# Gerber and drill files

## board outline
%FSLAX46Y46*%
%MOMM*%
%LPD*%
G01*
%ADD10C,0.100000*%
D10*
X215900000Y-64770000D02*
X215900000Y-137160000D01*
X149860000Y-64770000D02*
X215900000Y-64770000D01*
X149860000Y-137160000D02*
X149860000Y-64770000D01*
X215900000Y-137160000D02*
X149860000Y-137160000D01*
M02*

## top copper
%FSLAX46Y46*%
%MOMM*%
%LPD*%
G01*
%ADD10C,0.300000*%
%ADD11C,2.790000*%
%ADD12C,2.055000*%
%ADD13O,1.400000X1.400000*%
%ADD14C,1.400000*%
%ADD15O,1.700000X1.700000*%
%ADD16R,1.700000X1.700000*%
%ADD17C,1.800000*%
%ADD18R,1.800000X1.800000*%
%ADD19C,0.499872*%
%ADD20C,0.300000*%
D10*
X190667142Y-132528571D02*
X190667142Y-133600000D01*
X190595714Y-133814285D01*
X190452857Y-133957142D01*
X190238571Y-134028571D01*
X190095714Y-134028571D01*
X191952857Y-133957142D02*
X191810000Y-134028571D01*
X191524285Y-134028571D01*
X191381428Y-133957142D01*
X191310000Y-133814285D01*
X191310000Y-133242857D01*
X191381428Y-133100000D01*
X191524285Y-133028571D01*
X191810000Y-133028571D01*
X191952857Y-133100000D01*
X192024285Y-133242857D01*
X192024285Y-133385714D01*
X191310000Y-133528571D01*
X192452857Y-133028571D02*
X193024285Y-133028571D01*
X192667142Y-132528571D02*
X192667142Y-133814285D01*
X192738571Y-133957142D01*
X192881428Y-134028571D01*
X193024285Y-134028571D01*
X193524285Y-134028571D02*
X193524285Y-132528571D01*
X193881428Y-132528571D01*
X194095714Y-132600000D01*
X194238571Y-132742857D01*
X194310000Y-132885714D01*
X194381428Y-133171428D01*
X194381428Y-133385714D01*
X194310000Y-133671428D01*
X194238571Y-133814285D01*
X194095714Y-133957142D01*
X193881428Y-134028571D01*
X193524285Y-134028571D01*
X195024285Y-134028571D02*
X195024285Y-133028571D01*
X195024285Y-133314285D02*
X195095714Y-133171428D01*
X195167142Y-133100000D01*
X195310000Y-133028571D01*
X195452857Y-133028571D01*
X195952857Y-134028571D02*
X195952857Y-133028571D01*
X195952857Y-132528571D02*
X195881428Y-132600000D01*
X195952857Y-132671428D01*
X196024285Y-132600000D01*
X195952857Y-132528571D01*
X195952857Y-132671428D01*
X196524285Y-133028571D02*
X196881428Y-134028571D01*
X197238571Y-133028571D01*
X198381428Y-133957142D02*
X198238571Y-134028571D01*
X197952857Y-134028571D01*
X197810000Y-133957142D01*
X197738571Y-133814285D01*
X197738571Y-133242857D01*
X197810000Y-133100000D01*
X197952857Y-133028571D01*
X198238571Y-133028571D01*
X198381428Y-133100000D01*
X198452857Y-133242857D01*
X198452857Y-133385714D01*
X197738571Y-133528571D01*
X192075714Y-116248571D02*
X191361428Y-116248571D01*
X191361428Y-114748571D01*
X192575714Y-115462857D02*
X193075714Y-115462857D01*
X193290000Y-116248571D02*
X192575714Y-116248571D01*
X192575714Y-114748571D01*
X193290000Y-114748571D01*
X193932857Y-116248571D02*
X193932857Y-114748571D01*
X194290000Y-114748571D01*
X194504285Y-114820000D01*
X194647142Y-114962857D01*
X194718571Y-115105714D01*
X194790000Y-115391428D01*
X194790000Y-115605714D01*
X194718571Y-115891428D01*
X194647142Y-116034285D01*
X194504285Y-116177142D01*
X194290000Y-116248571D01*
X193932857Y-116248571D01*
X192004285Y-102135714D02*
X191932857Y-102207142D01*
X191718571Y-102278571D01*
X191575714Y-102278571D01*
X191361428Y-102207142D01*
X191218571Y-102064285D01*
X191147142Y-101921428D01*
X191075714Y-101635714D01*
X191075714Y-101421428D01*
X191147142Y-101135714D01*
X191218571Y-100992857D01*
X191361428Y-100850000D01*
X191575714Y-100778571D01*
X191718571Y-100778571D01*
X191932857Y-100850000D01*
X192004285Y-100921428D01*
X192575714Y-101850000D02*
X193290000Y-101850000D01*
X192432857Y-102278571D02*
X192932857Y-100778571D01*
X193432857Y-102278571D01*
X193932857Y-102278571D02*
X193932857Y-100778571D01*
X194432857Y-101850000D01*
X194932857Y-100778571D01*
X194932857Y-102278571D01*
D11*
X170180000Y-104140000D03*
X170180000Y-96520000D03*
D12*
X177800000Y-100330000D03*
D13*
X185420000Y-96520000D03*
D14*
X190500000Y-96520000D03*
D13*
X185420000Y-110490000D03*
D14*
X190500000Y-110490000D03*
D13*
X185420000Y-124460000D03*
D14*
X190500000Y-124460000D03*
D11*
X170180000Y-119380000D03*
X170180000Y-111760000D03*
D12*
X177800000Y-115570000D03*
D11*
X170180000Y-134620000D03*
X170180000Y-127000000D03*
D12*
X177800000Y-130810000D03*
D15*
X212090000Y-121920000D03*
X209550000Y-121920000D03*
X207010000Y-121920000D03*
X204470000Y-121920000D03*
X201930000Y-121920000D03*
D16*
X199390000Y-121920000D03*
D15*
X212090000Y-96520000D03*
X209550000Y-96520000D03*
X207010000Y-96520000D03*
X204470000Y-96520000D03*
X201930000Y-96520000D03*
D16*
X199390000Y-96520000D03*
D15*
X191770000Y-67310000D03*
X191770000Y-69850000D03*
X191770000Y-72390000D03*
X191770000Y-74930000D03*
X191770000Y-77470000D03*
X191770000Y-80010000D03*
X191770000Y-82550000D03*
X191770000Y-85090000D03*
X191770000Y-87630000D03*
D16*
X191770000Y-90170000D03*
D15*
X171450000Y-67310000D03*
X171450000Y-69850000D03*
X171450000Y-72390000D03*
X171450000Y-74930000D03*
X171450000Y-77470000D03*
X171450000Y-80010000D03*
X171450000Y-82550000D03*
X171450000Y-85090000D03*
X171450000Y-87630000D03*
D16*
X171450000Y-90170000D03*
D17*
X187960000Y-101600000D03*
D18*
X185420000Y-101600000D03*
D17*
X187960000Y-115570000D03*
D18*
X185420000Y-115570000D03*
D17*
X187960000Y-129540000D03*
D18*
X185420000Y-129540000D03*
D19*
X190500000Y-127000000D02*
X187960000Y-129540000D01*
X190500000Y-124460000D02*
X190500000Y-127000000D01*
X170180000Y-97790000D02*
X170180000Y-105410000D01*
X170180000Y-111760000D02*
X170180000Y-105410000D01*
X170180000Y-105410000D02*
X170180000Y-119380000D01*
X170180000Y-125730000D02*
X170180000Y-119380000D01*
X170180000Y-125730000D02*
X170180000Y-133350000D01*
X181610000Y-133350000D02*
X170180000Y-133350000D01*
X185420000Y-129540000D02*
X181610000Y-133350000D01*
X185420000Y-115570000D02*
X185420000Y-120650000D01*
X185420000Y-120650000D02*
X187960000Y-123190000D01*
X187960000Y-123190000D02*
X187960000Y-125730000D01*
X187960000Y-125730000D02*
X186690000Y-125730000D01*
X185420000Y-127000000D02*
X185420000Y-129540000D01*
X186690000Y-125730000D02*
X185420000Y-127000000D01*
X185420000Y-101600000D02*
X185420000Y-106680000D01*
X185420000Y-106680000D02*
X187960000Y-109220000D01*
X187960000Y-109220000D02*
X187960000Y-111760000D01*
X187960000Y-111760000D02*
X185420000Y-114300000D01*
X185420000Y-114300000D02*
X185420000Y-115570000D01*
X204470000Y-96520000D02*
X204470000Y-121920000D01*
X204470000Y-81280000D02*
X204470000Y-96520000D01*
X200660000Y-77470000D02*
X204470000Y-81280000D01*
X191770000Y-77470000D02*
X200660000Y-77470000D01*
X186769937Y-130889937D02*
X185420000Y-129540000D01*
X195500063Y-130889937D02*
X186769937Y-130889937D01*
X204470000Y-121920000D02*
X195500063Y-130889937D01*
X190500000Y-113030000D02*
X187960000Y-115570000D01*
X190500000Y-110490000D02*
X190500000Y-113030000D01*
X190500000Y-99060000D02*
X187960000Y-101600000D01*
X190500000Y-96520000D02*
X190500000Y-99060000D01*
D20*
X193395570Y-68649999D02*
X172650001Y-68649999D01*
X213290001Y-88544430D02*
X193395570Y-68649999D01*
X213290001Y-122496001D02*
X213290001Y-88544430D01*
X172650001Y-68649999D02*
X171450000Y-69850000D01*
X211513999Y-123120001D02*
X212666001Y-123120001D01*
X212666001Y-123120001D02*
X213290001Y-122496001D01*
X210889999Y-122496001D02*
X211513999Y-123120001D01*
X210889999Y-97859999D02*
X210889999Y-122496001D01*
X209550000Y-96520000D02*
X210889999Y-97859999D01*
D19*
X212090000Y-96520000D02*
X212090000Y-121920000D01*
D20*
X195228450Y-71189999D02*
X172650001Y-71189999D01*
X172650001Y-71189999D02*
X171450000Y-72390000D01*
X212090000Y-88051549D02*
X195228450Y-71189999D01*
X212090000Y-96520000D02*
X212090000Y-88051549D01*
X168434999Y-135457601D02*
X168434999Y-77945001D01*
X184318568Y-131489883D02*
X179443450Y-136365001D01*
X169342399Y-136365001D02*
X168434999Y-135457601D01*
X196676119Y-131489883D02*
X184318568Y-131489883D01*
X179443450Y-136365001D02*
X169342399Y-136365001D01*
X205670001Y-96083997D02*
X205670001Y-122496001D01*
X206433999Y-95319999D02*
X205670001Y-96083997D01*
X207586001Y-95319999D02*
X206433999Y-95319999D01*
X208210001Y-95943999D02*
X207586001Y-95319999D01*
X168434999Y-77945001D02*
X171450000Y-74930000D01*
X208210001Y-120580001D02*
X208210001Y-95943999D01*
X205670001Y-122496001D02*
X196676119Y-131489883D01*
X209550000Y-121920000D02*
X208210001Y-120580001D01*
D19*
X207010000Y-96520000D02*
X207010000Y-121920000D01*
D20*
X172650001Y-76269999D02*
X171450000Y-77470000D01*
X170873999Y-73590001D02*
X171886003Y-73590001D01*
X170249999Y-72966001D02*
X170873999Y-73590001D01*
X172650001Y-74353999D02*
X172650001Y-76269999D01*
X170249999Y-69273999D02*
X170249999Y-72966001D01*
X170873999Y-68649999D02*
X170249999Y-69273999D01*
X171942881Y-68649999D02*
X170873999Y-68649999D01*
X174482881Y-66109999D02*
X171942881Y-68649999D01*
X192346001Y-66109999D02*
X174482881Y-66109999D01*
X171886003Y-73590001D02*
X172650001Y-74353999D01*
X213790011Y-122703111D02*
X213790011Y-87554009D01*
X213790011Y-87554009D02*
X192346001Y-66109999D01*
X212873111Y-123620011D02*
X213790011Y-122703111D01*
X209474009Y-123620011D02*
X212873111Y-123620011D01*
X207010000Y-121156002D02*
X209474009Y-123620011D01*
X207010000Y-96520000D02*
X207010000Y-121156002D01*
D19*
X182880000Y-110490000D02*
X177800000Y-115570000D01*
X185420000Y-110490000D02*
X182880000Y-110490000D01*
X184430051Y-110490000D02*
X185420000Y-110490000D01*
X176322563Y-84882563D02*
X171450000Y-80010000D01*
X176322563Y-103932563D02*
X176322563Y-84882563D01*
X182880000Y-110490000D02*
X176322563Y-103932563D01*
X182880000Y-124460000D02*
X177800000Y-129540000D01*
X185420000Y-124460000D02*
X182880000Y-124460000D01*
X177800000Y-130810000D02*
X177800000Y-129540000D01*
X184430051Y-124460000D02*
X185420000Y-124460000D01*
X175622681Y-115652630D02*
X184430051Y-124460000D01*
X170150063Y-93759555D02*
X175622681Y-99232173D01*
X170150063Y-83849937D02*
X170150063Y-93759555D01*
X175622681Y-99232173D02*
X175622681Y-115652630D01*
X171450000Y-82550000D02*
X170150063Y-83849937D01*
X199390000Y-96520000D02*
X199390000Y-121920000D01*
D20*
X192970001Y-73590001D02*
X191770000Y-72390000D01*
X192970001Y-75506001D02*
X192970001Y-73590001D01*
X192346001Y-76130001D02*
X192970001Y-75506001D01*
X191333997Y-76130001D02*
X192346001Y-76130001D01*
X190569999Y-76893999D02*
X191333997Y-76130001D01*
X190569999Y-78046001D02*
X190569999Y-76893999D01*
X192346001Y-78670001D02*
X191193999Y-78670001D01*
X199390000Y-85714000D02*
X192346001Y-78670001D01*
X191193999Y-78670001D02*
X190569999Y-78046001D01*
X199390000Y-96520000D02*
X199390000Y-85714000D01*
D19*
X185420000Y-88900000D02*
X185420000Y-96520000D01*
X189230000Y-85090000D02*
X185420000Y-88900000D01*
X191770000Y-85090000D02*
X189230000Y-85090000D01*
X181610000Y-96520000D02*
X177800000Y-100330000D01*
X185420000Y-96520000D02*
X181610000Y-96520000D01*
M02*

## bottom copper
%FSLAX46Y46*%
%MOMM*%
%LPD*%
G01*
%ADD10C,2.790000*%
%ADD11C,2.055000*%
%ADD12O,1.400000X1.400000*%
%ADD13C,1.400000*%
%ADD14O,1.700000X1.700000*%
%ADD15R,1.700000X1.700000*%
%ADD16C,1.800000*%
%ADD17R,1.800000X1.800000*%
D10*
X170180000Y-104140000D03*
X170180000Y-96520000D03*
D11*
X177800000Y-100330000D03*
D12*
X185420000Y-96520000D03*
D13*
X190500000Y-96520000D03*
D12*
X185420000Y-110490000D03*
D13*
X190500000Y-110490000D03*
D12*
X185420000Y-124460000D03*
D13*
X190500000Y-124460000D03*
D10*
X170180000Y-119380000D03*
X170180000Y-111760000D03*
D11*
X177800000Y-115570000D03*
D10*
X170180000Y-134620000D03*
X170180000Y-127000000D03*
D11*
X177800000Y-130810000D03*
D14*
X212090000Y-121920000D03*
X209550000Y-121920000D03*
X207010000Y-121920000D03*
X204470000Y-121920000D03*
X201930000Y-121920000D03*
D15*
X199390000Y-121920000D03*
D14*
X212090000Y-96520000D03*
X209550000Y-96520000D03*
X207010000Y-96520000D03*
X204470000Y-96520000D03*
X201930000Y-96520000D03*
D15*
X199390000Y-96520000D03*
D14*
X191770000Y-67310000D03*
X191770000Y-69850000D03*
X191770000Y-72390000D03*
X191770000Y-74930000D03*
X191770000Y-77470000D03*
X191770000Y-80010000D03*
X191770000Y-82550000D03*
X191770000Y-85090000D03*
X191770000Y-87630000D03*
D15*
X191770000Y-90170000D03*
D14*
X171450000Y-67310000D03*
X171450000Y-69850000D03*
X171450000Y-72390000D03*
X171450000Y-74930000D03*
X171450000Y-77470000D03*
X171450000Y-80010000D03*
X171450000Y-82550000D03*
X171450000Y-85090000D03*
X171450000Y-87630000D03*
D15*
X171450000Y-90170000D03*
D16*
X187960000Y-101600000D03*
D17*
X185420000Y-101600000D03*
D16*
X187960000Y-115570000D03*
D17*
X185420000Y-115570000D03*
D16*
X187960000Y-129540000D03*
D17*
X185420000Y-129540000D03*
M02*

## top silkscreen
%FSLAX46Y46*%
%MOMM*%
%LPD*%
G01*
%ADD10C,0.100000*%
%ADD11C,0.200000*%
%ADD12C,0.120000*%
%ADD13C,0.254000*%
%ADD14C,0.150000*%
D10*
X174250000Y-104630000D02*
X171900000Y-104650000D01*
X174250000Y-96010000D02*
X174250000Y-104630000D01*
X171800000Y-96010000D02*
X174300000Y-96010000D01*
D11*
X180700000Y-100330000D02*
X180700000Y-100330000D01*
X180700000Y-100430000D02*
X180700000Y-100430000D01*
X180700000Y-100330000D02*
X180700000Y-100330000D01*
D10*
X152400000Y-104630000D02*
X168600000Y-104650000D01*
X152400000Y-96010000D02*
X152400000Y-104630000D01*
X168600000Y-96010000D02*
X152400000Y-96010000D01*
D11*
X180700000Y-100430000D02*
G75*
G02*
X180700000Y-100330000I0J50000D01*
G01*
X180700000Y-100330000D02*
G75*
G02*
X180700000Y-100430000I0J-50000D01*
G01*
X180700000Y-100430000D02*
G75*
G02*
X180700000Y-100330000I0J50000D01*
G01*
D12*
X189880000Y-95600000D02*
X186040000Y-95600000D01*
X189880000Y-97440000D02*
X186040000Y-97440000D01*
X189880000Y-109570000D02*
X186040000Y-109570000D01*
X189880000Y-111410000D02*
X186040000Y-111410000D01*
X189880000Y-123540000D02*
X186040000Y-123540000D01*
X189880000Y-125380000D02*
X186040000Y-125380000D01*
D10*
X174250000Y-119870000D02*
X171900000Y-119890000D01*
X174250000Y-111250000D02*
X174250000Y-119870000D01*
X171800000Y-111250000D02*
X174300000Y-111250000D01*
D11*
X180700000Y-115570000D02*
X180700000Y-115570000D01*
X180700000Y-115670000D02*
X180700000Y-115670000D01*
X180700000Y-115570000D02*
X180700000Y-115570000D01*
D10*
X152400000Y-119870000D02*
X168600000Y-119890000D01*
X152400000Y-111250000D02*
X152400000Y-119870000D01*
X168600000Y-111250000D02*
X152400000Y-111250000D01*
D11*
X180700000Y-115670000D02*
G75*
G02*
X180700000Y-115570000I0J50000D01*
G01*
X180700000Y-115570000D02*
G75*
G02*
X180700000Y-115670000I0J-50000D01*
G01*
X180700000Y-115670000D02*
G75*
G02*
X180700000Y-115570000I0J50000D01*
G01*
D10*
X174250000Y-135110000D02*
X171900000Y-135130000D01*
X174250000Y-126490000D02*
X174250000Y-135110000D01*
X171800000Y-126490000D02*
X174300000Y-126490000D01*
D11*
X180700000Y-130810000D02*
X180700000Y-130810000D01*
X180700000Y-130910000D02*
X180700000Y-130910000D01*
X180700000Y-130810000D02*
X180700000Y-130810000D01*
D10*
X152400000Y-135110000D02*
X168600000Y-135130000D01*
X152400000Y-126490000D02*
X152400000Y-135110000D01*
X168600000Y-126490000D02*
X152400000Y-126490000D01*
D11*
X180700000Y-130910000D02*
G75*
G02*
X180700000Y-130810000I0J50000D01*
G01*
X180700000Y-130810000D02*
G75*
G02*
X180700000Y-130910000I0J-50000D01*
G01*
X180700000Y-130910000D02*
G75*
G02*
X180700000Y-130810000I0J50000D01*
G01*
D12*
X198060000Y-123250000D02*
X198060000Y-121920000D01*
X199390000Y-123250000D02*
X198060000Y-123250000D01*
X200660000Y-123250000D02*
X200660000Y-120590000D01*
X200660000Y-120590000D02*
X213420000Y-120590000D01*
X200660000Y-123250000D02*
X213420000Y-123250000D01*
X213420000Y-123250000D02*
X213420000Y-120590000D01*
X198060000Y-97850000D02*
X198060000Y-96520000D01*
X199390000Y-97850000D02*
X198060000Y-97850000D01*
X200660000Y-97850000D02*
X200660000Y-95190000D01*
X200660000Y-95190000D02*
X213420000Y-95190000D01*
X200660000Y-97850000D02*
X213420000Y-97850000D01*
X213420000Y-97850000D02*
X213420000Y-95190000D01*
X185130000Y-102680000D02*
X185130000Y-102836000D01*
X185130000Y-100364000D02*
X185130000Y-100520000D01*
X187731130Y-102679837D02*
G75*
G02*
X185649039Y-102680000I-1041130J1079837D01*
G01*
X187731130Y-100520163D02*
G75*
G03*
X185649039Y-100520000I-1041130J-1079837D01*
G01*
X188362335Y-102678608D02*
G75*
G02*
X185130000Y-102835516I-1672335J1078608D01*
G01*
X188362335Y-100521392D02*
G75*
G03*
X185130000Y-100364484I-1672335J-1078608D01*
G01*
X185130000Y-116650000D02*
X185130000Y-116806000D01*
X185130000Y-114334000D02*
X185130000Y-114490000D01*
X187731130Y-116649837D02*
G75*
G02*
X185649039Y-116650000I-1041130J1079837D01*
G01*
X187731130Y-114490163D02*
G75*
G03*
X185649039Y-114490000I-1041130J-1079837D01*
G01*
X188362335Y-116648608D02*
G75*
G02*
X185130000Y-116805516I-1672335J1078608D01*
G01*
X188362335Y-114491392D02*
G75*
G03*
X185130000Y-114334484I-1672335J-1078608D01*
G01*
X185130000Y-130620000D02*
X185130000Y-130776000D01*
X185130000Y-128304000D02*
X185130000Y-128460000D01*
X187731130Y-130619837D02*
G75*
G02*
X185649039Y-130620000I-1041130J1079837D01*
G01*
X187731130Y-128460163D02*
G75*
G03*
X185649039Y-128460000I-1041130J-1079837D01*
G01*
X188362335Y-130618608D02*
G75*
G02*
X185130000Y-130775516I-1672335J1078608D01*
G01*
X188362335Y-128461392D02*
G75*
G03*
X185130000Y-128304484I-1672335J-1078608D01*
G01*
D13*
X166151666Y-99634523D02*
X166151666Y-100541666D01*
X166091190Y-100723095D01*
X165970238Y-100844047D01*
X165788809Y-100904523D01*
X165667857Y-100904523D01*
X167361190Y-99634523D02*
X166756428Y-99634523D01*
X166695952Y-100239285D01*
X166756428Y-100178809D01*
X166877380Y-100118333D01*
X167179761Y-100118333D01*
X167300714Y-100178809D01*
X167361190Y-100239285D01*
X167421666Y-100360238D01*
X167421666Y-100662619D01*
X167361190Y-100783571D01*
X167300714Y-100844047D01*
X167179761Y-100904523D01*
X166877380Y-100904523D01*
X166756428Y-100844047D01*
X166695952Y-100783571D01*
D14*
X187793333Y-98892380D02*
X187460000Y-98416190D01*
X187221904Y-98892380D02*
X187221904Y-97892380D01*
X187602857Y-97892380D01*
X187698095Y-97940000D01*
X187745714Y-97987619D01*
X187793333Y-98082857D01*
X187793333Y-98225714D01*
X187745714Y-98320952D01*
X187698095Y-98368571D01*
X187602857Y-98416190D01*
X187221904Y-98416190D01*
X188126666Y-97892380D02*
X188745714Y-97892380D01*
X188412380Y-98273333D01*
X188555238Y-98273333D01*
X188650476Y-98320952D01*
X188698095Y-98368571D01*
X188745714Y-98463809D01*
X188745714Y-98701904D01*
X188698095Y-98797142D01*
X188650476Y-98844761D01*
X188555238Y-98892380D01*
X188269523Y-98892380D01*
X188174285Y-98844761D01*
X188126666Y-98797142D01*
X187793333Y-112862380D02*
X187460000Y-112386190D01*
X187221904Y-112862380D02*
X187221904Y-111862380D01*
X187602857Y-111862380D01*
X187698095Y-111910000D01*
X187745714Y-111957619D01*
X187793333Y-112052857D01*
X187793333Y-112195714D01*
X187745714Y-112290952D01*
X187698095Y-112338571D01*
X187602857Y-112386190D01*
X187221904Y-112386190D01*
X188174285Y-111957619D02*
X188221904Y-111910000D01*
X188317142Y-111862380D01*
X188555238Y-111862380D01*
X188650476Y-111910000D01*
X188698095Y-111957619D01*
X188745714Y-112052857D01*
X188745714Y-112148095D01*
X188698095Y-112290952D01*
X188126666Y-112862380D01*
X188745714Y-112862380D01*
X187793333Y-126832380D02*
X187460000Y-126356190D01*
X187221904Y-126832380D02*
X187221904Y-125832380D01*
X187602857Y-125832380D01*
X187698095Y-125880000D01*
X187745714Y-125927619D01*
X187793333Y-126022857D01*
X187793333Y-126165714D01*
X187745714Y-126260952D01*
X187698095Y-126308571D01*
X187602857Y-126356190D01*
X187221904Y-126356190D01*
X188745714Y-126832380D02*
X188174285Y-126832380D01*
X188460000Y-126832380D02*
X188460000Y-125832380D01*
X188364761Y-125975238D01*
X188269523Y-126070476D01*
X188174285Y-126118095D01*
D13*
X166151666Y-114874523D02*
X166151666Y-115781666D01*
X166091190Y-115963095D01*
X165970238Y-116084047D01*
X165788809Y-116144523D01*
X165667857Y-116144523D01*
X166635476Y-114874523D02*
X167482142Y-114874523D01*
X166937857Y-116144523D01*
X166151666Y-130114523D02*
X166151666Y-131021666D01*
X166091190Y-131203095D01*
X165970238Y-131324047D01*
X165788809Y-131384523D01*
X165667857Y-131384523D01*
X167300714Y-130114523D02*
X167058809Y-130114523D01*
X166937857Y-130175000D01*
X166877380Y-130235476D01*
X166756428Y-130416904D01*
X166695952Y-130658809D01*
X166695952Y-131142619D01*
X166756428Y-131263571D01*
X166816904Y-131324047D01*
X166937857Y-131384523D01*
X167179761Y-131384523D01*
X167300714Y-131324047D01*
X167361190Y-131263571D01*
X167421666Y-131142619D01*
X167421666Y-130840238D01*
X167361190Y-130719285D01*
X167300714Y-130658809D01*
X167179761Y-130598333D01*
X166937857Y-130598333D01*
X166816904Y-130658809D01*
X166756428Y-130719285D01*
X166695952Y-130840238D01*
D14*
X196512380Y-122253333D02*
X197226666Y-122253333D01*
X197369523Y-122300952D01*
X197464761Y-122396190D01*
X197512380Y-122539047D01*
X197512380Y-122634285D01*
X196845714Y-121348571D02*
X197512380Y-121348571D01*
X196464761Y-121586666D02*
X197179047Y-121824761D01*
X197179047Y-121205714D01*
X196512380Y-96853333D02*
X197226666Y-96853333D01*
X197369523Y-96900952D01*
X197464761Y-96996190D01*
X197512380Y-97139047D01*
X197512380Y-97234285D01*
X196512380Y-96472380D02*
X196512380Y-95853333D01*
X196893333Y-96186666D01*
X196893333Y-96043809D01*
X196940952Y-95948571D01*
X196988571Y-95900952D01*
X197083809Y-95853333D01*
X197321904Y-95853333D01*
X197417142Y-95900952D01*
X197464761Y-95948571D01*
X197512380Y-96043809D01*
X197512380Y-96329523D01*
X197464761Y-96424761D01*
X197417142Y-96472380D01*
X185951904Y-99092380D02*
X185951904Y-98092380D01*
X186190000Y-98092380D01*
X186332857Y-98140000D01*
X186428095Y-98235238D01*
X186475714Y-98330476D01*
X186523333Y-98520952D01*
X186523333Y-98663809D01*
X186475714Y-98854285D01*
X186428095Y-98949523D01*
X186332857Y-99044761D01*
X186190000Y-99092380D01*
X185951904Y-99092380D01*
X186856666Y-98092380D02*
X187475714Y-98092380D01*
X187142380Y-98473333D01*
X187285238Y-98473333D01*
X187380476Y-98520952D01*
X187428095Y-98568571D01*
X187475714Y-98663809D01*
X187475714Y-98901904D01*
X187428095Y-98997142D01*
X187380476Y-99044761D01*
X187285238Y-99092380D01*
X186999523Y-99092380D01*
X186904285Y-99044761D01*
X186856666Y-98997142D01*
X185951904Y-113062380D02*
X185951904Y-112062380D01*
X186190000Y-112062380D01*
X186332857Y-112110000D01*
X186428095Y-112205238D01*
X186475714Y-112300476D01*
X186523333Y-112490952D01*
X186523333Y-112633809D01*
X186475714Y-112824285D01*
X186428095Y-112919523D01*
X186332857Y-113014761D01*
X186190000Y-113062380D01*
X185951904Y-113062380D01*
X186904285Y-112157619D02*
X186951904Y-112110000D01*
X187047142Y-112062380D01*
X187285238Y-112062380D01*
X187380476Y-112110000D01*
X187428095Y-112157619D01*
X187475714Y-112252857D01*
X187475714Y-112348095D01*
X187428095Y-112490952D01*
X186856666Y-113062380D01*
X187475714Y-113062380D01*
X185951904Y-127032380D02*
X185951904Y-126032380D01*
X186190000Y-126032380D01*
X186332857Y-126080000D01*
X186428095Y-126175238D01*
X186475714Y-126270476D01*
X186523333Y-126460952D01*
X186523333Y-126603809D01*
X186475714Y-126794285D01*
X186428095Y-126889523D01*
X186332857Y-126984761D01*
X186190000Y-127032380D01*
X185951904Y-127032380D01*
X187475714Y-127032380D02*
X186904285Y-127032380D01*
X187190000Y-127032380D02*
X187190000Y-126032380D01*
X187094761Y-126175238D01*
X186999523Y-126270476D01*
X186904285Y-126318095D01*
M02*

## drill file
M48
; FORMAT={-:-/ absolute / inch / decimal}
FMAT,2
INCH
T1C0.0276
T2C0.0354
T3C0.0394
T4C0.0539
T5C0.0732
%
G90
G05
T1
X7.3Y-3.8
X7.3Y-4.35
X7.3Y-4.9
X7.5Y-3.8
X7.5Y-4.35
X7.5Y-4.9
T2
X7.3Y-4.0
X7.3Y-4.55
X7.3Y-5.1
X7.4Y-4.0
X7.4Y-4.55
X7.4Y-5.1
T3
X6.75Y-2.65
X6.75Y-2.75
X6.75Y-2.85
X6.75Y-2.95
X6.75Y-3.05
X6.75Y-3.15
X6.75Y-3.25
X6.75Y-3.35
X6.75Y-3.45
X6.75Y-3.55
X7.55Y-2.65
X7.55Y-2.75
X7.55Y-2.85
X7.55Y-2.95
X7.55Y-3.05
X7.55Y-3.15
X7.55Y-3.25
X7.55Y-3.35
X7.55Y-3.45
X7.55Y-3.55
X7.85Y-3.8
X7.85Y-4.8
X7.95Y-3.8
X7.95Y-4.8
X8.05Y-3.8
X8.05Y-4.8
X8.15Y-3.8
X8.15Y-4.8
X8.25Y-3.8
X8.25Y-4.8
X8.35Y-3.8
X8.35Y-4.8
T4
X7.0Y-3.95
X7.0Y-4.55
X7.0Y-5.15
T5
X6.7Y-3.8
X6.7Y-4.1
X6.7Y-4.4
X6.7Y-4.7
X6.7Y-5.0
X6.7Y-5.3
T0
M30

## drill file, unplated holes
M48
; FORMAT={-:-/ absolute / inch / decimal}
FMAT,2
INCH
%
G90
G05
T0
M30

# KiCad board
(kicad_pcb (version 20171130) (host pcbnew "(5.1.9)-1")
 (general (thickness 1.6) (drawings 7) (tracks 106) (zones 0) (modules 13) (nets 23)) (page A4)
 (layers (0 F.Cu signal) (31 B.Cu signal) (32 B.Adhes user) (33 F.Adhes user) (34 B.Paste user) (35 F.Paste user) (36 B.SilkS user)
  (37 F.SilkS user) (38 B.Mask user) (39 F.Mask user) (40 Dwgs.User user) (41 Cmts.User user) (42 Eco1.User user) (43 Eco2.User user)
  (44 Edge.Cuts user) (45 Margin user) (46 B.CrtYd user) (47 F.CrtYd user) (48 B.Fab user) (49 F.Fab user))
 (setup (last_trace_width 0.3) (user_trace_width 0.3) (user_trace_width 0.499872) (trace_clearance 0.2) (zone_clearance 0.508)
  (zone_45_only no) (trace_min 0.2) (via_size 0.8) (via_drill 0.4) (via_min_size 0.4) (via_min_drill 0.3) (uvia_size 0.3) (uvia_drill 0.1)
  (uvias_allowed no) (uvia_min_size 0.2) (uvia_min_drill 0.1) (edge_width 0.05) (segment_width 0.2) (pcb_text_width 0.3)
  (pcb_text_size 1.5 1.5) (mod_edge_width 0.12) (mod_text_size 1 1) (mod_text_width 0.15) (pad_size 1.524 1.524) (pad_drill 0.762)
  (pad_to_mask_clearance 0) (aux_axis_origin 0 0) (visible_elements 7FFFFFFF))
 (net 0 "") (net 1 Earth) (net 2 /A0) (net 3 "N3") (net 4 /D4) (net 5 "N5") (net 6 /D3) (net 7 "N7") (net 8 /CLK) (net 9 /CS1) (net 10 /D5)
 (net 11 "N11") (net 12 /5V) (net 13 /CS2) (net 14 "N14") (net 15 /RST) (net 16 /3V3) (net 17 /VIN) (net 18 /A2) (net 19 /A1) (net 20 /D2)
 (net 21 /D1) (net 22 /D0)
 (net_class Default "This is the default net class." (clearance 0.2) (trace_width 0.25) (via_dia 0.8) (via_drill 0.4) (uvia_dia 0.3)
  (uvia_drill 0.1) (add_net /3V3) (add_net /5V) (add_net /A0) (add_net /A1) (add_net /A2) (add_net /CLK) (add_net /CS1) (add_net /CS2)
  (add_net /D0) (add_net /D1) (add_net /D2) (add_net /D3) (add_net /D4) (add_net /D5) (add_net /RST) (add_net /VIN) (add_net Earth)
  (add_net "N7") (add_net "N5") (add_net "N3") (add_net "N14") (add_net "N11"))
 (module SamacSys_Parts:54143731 (layer F.Cu) (at 177.8 100.33)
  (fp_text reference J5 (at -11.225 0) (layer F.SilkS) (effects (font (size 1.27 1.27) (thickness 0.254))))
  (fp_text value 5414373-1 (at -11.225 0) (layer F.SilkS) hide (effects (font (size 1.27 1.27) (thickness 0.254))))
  (fp_line (start -3.55 4.3) (end -5.9 4.32) (layer F.SilkS) (width 0.1))
  (fp_line (start -3.55 -4.32) (end -3.55 4.3) (layer F.SilkS) (width 0.1))
  (fp_line (start -6 -4.32) (end -3.5 -4.32) (layer F.SilkS) (width 0.1))
  (fp_line (start 2.9 0) (end 2.9 0) (layer F.SilkS) (width 0.2))
  (fp_line (start 2.9 0.1) (end 2.9 0.1) (layer F.SilkS) (width 0.2))
  (fp_line (start 2.9 0) (end 2.9 0) (layer F.SilkS) (width 0.2))
  (fp_line (start -25.4 4.3) (end -9.2 4.32) (layer F.SilkS) (width 0.1))
  (fp_line (start -25.4 -4.32) (end -25.4 4.3) (layer F.SilkS) (width 0.1))
  (fp_line (start -9.2 -4.32) (end -25.4 -4.32) (layer F.SilkS) (width 0.1))
  (fp_arc (start 2.9 0.05) (end 2.9 0) (angle -180) (layer F.SilkS) (width 0.2))
  (fp_arc (start 2.9 0.05) (end 2.9 0.1) (angle -180) (layer F.SilkS) (width 0.2))
  (fp_arc (start 2.9 0.05) (end 2.9 0) (angle -180) (layer F.SilkS) (width 0.2))
  (pad 3 thru_hole circle (at -7.62 3.81) (size 2.79 2.79) (drill 1.86) (layers *.Cu *.Mask) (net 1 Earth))
  (pad 2 thru_hole circle (at -7.62 -3.81) (size 2.79 2.79) (drill 1.86) (layers *.Cu *.Mask) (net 1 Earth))
  (pad 1 thru_hole circle (at 0 0) (size 2.055 2.055) (drill 1.37) (layers *.Cu *.Mask) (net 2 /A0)))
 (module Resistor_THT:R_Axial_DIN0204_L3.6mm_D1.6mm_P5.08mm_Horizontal (layer F.Cu) (at 190.5 96.52 180)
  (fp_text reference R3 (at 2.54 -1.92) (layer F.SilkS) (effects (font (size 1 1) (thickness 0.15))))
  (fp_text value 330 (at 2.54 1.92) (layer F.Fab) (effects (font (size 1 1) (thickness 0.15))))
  (fp_line (start 0.62 0.92) (end 4.46 0.92) (layer F.SilkS) (width 0.12))
  (fp_line (start 0.62 -0.92) (end 4.46 -0.92) (layer F.SilkS) (width 0.12))
  (pad 2 thru_hole oval (at 5.08 0 180) (size 1.4 1.4) (drill 0.7) (layers *.Cu *.Mask) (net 2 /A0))
  (pad 1 thru_hole circle (at 0 0 180) (size 1.4 1.4) (drill 0.7) (layers *.Cu *.Mask) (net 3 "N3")))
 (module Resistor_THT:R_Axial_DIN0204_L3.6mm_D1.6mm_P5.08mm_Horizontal (layer F.Cu) (at 190.5 110.49 180)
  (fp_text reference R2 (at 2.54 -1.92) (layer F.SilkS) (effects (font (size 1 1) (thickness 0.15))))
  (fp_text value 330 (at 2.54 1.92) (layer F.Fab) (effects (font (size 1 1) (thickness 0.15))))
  (fp_line (start 0.62 0.92) (end 4.46 0.92) (layer F.SilkS) (width 0.12))
  (fp_line (start 0.62 -0.92) (end 4.46 -0.92) (layer F.SilkS) (width 0.12))
  (pad 2 thru_hole oval (at 5.08 0 180) (size 1.4 1.4) (drill 0.7) (layers *.Cu *.Mask) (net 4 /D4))
  (pad 1 thru_hole circle (at 0 0 180) (size 1.4 1.4) (drill 0.7) (layers *.Cu *.Mask) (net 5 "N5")))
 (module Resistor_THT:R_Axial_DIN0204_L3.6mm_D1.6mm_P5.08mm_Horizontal (layer F.Cu) (at 190.5 124.46 180)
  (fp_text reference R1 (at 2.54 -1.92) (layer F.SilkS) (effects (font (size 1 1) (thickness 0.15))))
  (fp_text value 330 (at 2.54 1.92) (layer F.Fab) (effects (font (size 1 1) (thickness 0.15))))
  (fp_line (start 0.62 0.92) (end 4.46 0.92) (layer F.SilkS) (width 0.12))
  (fp_line (start 0.62 -0.92) (end 4.46 -0.92) (layer F.SilkS) (width 0.12))
  (pad 2 thru_hole oval (at 5.08 0 180) (size 1.4 1.4) (drill 0.7) (layers *.Cu *.Mask) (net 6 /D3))
  (pad 1 thru_hole circle (at 0 0 180) (size 1.4 1.4) (drill 0.7) (layers *.Cu *.Mask) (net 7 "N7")))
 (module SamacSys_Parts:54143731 (layer F.Cu) (at 177.8 115.57)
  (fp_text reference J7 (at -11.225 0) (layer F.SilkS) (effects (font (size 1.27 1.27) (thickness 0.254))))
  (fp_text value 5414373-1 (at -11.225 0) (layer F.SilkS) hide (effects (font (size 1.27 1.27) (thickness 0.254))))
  (fp_line (start -3.55 4.3) (end -5.9 4.32) (layer F.SilkS) (width 0.1))
  (fp_line (start -3.55 -4.32) (end -3.55 4.3) (layer F.SilkS) (width 0.1))
  (fp_line (start -6 -4.32) (end -3.5 -4.32) (layer F.SilkS) (width 0.1))
  (fp_line (start 2.9 0) (end 2.9 0) (layer F.SilkS) (width 0.2))
  (fp_line (start 2.9 0.1) (end 2.9 0.1) (layer F.SilkS) (width 0.2))
  (fp_line (start 2.9 0) (end 2.9 0) (layer F.SilkS) (width 0.2))
  (fp_line (start -25.4 4.3) (end -9.2 4.32) (layer F.SilkS) (width 0.1))
  (fp_line (start -25.4 -4.32) (end -25.4 4.3) (layer F.SilkS) (width 0.1))
  (fp_line (start -9.2 -4.32) (end -25.4 -4.32) (layer F.SilkS) (width 0.1))
  (fp_arc (start 2.9 0.05) (end 2.9 0) (angle -180) (layer F.SilkS) (width 0.2))
  (fp_arc (start 2.9 0.05) (end 2.9 0.1) (angle -180) (layer F.SilkS) (width 0.2))
  (fp_arc (start 2.9 0.05) (end 2.9 0) (angle -180) (layer F.SilkS) (width 0.2))
  (pad 3 thru_hole circle (at -7.62 3.81) (size 2.79 2.79) (drill 1.86) (layers *.Cu *.Mask) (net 1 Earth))
  (pad 2 thru_hole circle (at -7.62 -3.81) (size 2.79 2.79) (drill 1.86) (layers *.Cu *.Mask) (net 1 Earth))
  (pad 1 thru_hole circle (at 0 0) (size 2.055 2.055) (drill 1.37) (layers *.Cu *.Mask) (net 4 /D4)))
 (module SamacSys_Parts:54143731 (layer F.Cu) (at 177.8 130.81)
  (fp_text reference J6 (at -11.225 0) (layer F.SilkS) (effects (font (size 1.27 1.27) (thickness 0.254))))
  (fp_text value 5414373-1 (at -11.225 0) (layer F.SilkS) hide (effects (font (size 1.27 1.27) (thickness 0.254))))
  (fp_line (start -3.55 4.3) (end -5.9 4.32) (layer F.SilkS) (width 0.1))
  (fp_line (start -3.55 -4.32) (end -3.55 4.3) (layer F.SilkS) (width 0.1))
  (fp_line (start -6 -4.32) (end -3.5 -4.32) (layer F.SilkS) (width 0.1))
  (fp_line (start 2.9 0) (end 2.9 0) (layer F.SilkS) (width 0.2))
  (fp_line (start 2.9 0.1) (end 2.9 0.1) (layer F.SilkS) (width 0.2))
  (fp_line (start 2.9 0) (end 2.9 0) (layer F.SilkS) (width 0.2))
  (fp_line (start -25.4 4.3) (end -9.2 4.32) (layer F.SilkS) (width 0.1))
  (fp_line (start -25.4 -4.32) (end -25.4 4.3) (layer F.SilkS) (width 0.1))
  (fp_line (start -9.2 -4.32) (end -25.4 -4.32) (layer F.SilkS) (width 0.1))
  (fp_arc (start 2.9 0.05) (end 2.9 0) (angle -180) (layer F.SilkS) (width 0.2))
  (fp_arc (start 2.9 0.05) (end 2.9 0.1) (angle -180) (layer F.SilkS) (width 0.2))
  (fp_arc (start 2.9 0.05) (end 2.9 0) (angle -180) (layer F.SilkS) (width 0.2))
  (pad 3 thru_hole circle (at -7.62 3.81) (size 2.79 2.79) (drill 1.86) (layers *.Cu *.Mask) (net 1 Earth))
  (pad 2 thru_hole circle (at -7.62 -3.81) (size 2.79 2.79) (drill 1.86) (layers *.Cu *.Mask) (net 1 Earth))
  (pad 1 thru_hole circle (at 0 0) (size 2.055 2.055) (drill 1.37) (layers *.Cu *.Mask) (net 6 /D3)))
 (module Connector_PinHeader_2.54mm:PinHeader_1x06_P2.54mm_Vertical (layer F.Cu) (at 199.39 121.92 90)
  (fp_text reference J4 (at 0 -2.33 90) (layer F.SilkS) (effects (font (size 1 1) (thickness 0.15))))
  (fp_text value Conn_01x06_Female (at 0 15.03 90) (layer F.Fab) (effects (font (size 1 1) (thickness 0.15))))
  (fp_line (start -1.33 -1.33) (end 0 -1.33) (layer F.SilkS) (width 0.12))
  (fp_line (start -1.33 0) (end -1.33 -1.33) (layer F.SilkS) (width 0.12))
  (fp_line (start -1.33 1.27) (end 1.33 1.27) (layer F.SilkS) (width 0.12))
  (fp_line (start 1.33 1.27) (end 1.33 14.03) (layer F.SilkS) (width 0.12))
  (fp_line (start -1.33 1.27) (end -1.33 14.03) (layer F.SilkS) (width 0.12))
  (fp_line (start -1.33 14.03) (end 1.33 14.03) (layer F.SilkS) (width 0.12))
  (pad 6 thru_hole oval (at 0 12.7 90) (size 1.7 1.7) (drill 1) (layers *.Cu *.Mask) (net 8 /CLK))
  (pad 5 thru_hole oval (at 0 10.16 90) (size 1.7 1.7) (drill 1) (layers *.Cu *.Mask) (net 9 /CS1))
  (pad 4 thru_hole oval (at 0 7.62 90) (size 1.7 1.7) (drill 1) (layers *.Cu *.Mask) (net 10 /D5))
  (pad 3 thru_hole oval (at 0 5.08 90) (size 1.7 1.7) (drill 1) (layers *.Cu *.Mask) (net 1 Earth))
  (pad 2 thru_hole oval (at 0 2.54 90) (size 1.7 1.7) (drill 1) (layers *.Cu *.Mask) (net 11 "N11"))
  (pad 1 thru_hole rect (at 0 0 90) (size 1.7 1.7) (drill 1) (layers *.Cu *.Mask) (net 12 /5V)))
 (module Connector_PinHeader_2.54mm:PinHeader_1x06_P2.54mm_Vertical (layer F.Cu) (at 199.39 96.52 90)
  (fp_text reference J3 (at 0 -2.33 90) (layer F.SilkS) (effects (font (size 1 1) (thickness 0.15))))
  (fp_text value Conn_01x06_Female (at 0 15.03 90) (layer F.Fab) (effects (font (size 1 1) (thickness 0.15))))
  (fp_line (start -1.33 -1.33) (end 0 -1.33) (layer F.SilkS) (width 0.12))
  (fp_line (start -1.33 0) (end -1.33 -1.33) (layer F.SilkS) (width 0.12))
  (fp_line (start -1.33 1.27) (end 1.33 1.27) (layer F.SilkS) (width 0.12))
  (fp_line (start 1.33 1.27) (end 1.33 14.03) (layer F.SilkS) (width 0.12))
  (fp_line (start -1.33 1.27) (end -1.33 14.03) (layer F.SilkS) (width 0.12))
  (fp_line (start -1.33 14.03) (end 1.33 14.03) (layer F.SilkS) (width 0.12))
  (pad 6 thru_hole oval (at 0 12.7 90) (size 1.7 1.7) (drill 1) (layers *.Cu *.Mask) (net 8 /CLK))
  (pad 5 thru_hole oval (at 0 10.16 90) (size 1.7 1.7) (drill 1) (layers *.Cu *.Mask) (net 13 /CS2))
  (pad 4 thru_hole oval (at 0 7.62 90) (size 1.7 1.7) (drill 1) (layers *.Cu *.Mask) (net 10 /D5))
  (pad 3 thru_hole oval (at 0 5.08 90) (size 1.7 1.7) (drill 1) (layers *.Cu *.Mask) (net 1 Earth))
  (pad 2 thru_hole oval (at 0 2.54 90) (size 1.7 1.7) (drill 1) (layers *.Cu *.Mask) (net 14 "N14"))
  (pad 1 thru_hole rect (at 0 0 90) (size 1.7 1.7) (drill 1) (layers *.Cu *.Mask) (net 12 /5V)))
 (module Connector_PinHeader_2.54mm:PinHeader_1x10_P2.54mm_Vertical (layer B.Cu) (at 191.77 90.17)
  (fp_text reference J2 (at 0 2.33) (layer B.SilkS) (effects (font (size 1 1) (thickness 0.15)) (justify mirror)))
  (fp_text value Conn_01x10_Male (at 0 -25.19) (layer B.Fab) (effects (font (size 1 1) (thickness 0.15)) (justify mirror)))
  (pad 10 thru_hole oval (at 0 -22.86) (size 1.7 1.7) (drill 1) (layers *.Cu *.Mask) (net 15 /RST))
  (pad 9 thru_hole oval (at 0 -20.32) (size 1.7 1.7) (drill 1) (layers *.Cu *.Mask) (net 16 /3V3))
  (pad 8 thru_hole oval (at 0 -17.78) (size 1.7 1.7) (drill 1) (layers *.Cu *.Mask) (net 12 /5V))
  (pad 7 thru_hole oval (at 0 -15.24) (size 1.7 1.7) (drill 1) (layers *.Cu *.Mask) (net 1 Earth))
  (pad 6 thru_hole oval (at 0 -12.7) (size 1.7 1.7) (drill 1) (layers *.Cu *.Mask) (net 1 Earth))
  (pad 5 thru_hole oval (at 0 -10.16) (size 1.7 1.7) (drill 1) (layers *.Cu *.Mask) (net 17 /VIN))
  (pad 4 thru_hole oval (at 0 -7.62) (size 1.7 1.7) (drill 1) (layers *.Cu *.Mask) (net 17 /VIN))
  (pad 3 thru_hole oval (at 0 -5.08) (size 1.7 1.7) (drill 1) (layers *.Cu *.Mask) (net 2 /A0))
  (pad 2 thru_hole oval (at 0 -2.54) (size 1.7 1.7) (drill 1) (layers *.Cu *.Mask) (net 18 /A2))
  (pad 1 thru_hole rect (at 0 0) (size 1.7 1.7) (drill 1) (layers *.Cu *.Mask) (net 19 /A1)))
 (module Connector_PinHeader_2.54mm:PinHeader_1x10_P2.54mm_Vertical (layer B.Cu) (at 171.45 90.17)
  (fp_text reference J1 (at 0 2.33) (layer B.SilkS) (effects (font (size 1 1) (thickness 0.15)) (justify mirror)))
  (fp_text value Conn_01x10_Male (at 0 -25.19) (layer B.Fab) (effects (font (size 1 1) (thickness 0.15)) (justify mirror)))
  (pad 10 thru_hole oval (at 0 -22.86) (size 1.7 1.7) (drill 1) (layers *.Cu *.Mask) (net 1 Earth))
  (pad 9 thru_hole oval (at 0 -20.32) (size 1.7 1.7) (drill 1) (layers *.Cu *.Mask) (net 13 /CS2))
  (pad 8 thru_hole oval (at 0 -17.78) (size 1.7 1.7) (drill 1) (layers *.Cu *.Mask) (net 8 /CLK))
  (pad 7 thru_hole oval (at 0 -15.24) (size 1.7 1.7) (drill 1) (layers *.Cu *.Mask) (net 9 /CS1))
  (pad 6 thru_hole oval (at 0 -12.7) (size 1.7 1.7) (drill 1) (layers *.Cu *.Mask) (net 10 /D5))
  (pad 5 thru_hole oval (at 0 -10.16) (size 1.7 1.7) (drill 1) (layers *.Cu *.Mask) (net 4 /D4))
  (pad 4 thru_hole oval (at 0 -7.62) (size 1.7 1.7) (drill 1) (layers *.Cu *.Mask) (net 6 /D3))
  (pad 3 thru_hole oval (at 0 -5.08) (size 1.7 1.7) (drill 1) (layers *.Cu *.Mask) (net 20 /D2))
  (pad 2 thru_hole oval (at 0 -2.54) (size 1.7 1.7) (drill 1) (layers *.Cu *.Mask) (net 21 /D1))
  (pad 1 thru_hole rect (at 0 0) (size 1.7 1.7) (drill 1) (layers *.Cu *.Mask) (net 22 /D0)))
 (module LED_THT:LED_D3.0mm (layer F.Cu) (at 185.42 101.6)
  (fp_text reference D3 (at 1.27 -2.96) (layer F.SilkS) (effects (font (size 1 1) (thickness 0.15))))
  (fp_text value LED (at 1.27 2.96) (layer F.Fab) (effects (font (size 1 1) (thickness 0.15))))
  (fp_line (start -0.29 1.08) (end -0.29 1.236) (layer F.SilkS) (width 0.12))
  (fp_line (start -0.29 -1.236) (end -0.29 -1.08) (layer F.SilkS) (width 0.12))
  (fp_arc (start 1.27 0) (end 0.229039 1.08) (angle -87.9) (layer F.SilkS) (width 0.12))
  (fp_arc (start 1.27 0) (end 0.229039 -1.08) (angle 87.9) (layer F.SilkS) (width 0.12))
  (fp_arc (start 1.27 0) (end -0.29 1.235516) (angle -108.8) (layer F.SilkS) (width 0.12))
  (fp_arc (start 1.27 0) (end -0.29 -1.235516) (angle 108.8) (layer F.SilkS) (width 0.12))
  (pad 2 thru_hole circle (at 2.54 0) (size 1.8 1.8) (drill 0.9) (layers *.Cu *.Mask) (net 3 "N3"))
  (pad 1 thru_hole rect (at 0 0) (size 1.8 1.8) (drill 0.9) (layers *.Cu *.Mask) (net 1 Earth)))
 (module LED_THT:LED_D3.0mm (layer F.Cu) (at 185.42 115.57)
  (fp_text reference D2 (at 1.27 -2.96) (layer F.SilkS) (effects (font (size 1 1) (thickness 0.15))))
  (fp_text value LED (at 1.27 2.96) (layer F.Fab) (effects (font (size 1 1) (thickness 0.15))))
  (fp_line (start -0.29 1.08) (end -0.29 1.236) (layer F.SilkS) (width 0.12))
  (fp_line (start -0.29 -1.236) (end -0.29 -1.08) (layer F.SilkS) (width 0.12))
  (fp_arc (start 1.27 0) (end 0.229039 1.08) (angle -87.9) (layer F.SilkS) (width 0.12))
  (fp_arc (start 1.27 0) (end 0.229039 -1.08) (angle 87.9) (layer F.SilkS) (width 0.12))
  (fp_arc (start 1.27 0) (end -0.29 1.235516) (angle -108.8) (layer F.SilkS) (width 0.12))
  (fp_arc (start 1.27 0) (end -0.29 -1.235516) (angle 108.8) (layer F.SilkS) (width 0.12))
  (pad 2 thru_hole circle (at 2.54 0) (size 1.8 1.8) (drill 0.9) (layers *.Cu *.Mask) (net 5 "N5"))
  (pad 1 thru_hole rect (at 0 0) (size 1.8 1.8) (drill 0.9) (layers *.Cu *.Mask) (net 1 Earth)))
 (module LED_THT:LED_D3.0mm (layer F.Cu) (at 185.42 129.54)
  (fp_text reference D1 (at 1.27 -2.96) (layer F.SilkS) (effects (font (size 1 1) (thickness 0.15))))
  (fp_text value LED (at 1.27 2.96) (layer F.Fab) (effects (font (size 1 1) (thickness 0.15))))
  (fp_line (start -0.29 1.08) (end -0.29 1.236) (layer F.SilkS) (width 0.12))
  (fp_line (start -0.29 -1.236) (end -0.29 -1.08) (layer F.SilkS) (width 0.12))
  (fp_arc (start 1.27 0) (end 0.229039 1.08) (angle -87.9) (layer F.SilkS) (width 0.12))
  (fp_arc (start 1.27 0) (end 0.229039 -1.08) (angle 87.9) (layer F.SilkS) (width 0.12))
  (fp_arc (start 1.27 0) (end -0.29 1.235516) (angle -108.8) (layer F.SilkS) (width 0.12))
  (fp_arc (start 1.27 0) (end -0.29 -1.235516) (angle 108.8) (layer F.SilkS) (width 0.12))
  (pad 2 thru_hole circle (at 2.54 0) (size 1.8 1.8) (drill 0.9) (layers *.Cu *.Mask) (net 7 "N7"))
  (pad 1 thru_hole rect (at 0 0) (size 1.8 1.8) (drill 0.9) (layers *.Cu *.Mask) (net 1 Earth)))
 (gr_line (start 215.9 64.77) (end 215.9 137.16) (layer Edge.Cuts) (width 0.1))
 (gr_line (start 149.86 64.77) (end 215.9 64.77) (layer Edge.Cuts) (width 0.1))
 (gr_line (start 149.86 137.16) (end 149.86 64.77) (layer Edge.Cuts) (width 0.1))
 (gr_line (start 215.9 137.16) (end 149.86 137.16) (layer Edge.Cuts) (width 0.1))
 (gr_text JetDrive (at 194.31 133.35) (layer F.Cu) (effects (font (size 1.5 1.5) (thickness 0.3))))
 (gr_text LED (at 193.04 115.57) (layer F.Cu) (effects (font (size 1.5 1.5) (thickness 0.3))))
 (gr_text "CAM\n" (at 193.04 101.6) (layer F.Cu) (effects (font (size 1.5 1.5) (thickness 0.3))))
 (segment (start 190.5 127) (end 187.96 129.54) (width 0.499872) (layer F.Cu) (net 7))
 (segment (start 190.5 124.46) (end 190.5 127) (width 0.499872) (layer F.Cu) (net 7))
 (segment (start 170.18 97.79) (end 170.18 105.41) (width 0.499872) (layer F.Cu) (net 1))
 (segment (start 170.18 111.76) (end 170.18 105.41) (width 0.499872) (layer F.Cu) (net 1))
 (segment (start 170.18 105.41) (end 170.18 119.38) (width 0.499872) (layer F.Cu) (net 1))
 (segment (start 170.18 125.73) (end 170.18 119.38) (width 0.499872) (layer F.Cu) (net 1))
 (segment (start 170.18 125.73) (end 170.18 133.35) (width 0.499872) (layer F.Cu) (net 1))
 (segment (start 181.61 133.35) (end 170.18 133.35) (width 0.499872) (layer F.Cu) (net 1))
 (segment (start 185.42 129.54) (end 181.61 133.35) (width 0.499872) (layer F.Cu) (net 1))
 (segment (start 185.42 115.57) (end 185.42 120.65) (width 0.499872) (layer F.Cu) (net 1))
 (segment (start 185.42 120.65) (end 187.96 123.19) (width 0.499872) (layer F.Cu) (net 1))
 (segment (start 187.96 123.19) (end 187.96 125.73) (width 0.499872) (layer F.Cu) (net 1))
 (segment (start 187.96 125.73) (end 186.69 125.73) (width 0.499872) (layer F.Cu) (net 1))
 (segment (start 185.42 127) (end 185.42 129.54) (width 0.499872) (layer F.Cu) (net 1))
 (segment (start 186.69 125.73) (end 185.42 127) (width 0.499872) (layer F.Cu) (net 1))
 (segment (start 185.42 101.6) (end 185.42 106.68) (width 0.499872) (layer F.Cu) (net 1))
 (segment (start 185.42 106.68) (end 187.96 109.22) (width 0.499872) (layer F.Cu) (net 1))
 (segment (start 187.96 109.22) (end 187.96 111.76) (width 0.499872) (layer F.Cu) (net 1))
 (segment (start 187.96 111.76) (end 185.42 114.3) (width 0.499872) (layer F.Cu) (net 1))
 (segment (start 185.42 114.3) (end 185.42 115.57) (width 0.499872) (layer F.Cu) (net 1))
 (segment (start 204.47 96.52) (end 204.47 121.92) (width 0.499872) (layer F.Cu) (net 1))
 (segment (start 204.47 81.28) (end 204.47 96.52) (width 0.499872) (layer F.Cu) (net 1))
 (segment (start 200.66 77.47) (end 204.47 81.28) (width 0.499872) (layer F.Cu) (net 1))
 (segment (start 191.77 77.47) (end 200.66 77.47) (width 0.499872) (layer F.Cu) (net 1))
 (segment (start 186.769937 130.889937) (end 185.42 129.54) (width 0.499872) (layer F.Cu) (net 1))
 (segment (start 195.500063 130.889937) (end 186.769937 130.889937) (width 0.499872) (layer F.Cu) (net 1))
 (segment (start 204.47 121.92) (end 195.500063 130.889937) (width 0.499872) (layer F.Cu) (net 1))
 (segment (start 190.5 113.03) (end 187.96 115.57) (width 0.499872) (layer F.Cu) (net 5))
 (segment (start 190.5 110.49) (end 190.5 113.03) (width 0.499872) (layer F.Cu) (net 5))
 (segment (start 190.5 99.06) (end 187.96 101.6) (width 0.499872) (layer F.Cu) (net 3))
 (segment (start 190.5 96.52) (end 190.5 99.06) (width 0.499872) (layer F.Cu) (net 3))
 (segment (start 193.39557 68.649999) (end 172.650001 68.649999) (width 0.3) (layer F.Cu) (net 13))
 (segment (start 213.290001 88.54443) (end 193.39557 68.649999) (width 0.3) (layer F.Cu) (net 13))
 (segment (start 213.290001 122.496001) (end 213.290001 88.54443) (width 0.3) (layer F.Cu) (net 13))
 (segment (start 172.650001 68.649999) (end 171.45 69.85) (width 0.3) (layer F.Cu) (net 13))
 (segment (start 211.513999 123.120001) (end 212.666001 123.120001) (width 0.3) (layer F.Cu) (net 13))
 (segment (start 212.666001 123.120001) (end 213.290001 122.496001) (width 0.3) (layer F.Cu) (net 13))
 (segment (start 210.889999 122.496001) (end 211.513999 123.120001) (width 0.3) (layer F.Cu) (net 13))
 (segment (start 210.889999 97.859999) (end 210.889999 122.496001) (width 0.3) (layer F.Cu) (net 13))
 (segment (start 209.55 96.52) (end 210.889999 97.859999) (width 0.3) (layer F.Cu) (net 13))
 (segment (start 212.09 96.52) (end 212.09 121.92) (width 0.499872) (layer F.Cu) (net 8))
 (segment (start 195.22845 71.189999) (end 172.650001 71.189999) (width 0.3) (layer F.Cu) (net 8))
 (segment (start 172.650001 71.189999) (end 171.45 72.39) (width 0.3) (layer F.Cu) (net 8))
 (segment (start 212.09 88.051549) (end 195.22845 71.189999) (width 0.3) (layer F.Cu) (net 8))
 (segment (start 212.09 96.52) (end 212.09 88.051549) (width 0.3) (layer F.Cu) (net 8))
 (segment (start 168.434999 135.457601) (end 168.434999 77.945001) (width 0.3) (layer F.Cu) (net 9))
 (segment (start 184.318568 131.489883) (end 179.44345 136.365001) (width 0.3) (layer F.Cu) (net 9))
 (segment (start 169.342399 136.365001) (end 168.434999 135.457601) (width 0.3) (layer F.Cu) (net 9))
 (segment (start 196.676119 131.489883) (end 184.318568 131.489883) (width 0.3) (layer F.Cu) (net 9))
 (segment (start 179.44345 136.365001) (end 169.342399 136.365001) (width 0.3) (layer F.Cu) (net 9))
 (segment (start 205.670001 96.083997) (end 205.670001 122.496001) (width 0.3) (layer F.Cu) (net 9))
 (segment (start 206.433999 95.319999) (end 205.670001 96.083997) (width 0.3) (layer F.Cu) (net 9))
 (segment (start 207.586001 95.319999) (end 206.433999 95.319999) (width 0.3) (layer F.Cu) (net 9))
 (segment (start 208.210001 95.943999) (end 207.586001 95.319999) (width 0.3) (layer F.Cu) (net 9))
 (segment (start 168.434999 77.945001) (end 171.45 74.93) (width 0.3) (layer F.Cu) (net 9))
 (segment (start 208.210001 120.580001) (end 208.210001 95.943999) (width 0.3) (layer F.Cu) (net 9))
 (segment (start 205.670001 122.496001) (end 196.676119 131.489883) (width 0.3) (layer F.Cu) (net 9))
 (segment (start 209.55 121.92) (end 208.210001 120.580001) (width 0.3) (layer F.Cu) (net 9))
 (segment (start 207.01 96.52) (end 207.01 121.92) (width 0.499872) (layer F.Cu) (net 10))
 (segment (start 172.650001 76.269999) (end 171.45 77.47) (width 0.3) (layer F.Cu) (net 10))
 (segment (start 170.873999 73.590001) (end 171.886003 73.590001) (width 0.3) (layer F.Cu) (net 10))
 (segment (start 170.249999 72.966001) (end 170.873999 73.590001) (width 0.3) (layer F.Cu) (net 10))
 (segment (start 172.650001 74.353999) (end 172.650001 76.269999) (width 0.3) (layer F.Cu) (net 10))
 (segment (start 170.249999 69.273999) (end 170.249999 72.966001) (width 0.3) (layer F.Cu) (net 10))
 (segment (start 170.873999 68.649999) (end 170.249999 69.273999) (width 0.3) (layer F.Cu) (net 10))
 (segment (start 171.942881 68.649999) (end 170.873999 68.649999) (width 0.3) (layer F.Cu) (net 10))
 (segment (start 174.482881 66.109999) (end 171.942881 68.649999) (width 0.3) (layer F.Cu) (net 10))
 (segment (start 192.346001 66.109999) (end 174.482881 66.109999) (width 0.3) (layer F.Cu) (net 10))
 (segment (start 171.886003 73.590001) (end 172.650001 74.353999) (width 0.3) (layer F.Cu) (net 10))
 (segment (start 213.790011 122.703111) (end 213.790011 87.554009) (width 0.3) (layer F.Cu) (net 10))
 (segment (start 213.790011 87.554009) (end 192.346001 66.109999) (width 0.3) (layer F.Cu) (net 10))
 (segment (start 212.873111 123.620011) (end 213.790011 122.703111) (width 0.3) (layer F.Cu) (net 10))
 (segment (start 209.474009 123.620011) (end 212.873111 123.620011) (width 0.3) (layer F.Cu) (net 10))
 (segment (start 207.01 121.156002) (end 209.474009 123.620011) (width 0.3) (layer F.Cu) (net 10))
 (segment (start 207.01 96.52) (end 207.01 121.156002) (width 0.3) (layer F.Cu) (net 10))
 (segment (start 182.88 110.49) (end 177.8 115.57) (width 0.499872) (layer F.Cu) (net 4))
 (segment (start 185.42 110.49) (end 182.88 110.49) (width 0.499872) (layer F.Cu) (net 4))
 (segment (start 184.430051 110.49) (end 185.42 110.49) (width 0.499872) (layer F.Cu) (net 4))
 (segment (start 176.322563 84.882563) (end 171.45 80.01) (width 0.499872) (layer F.Cu) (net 4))
 (segment (start 176.322563 103.932563) (end 176.322563 84.882563) (width 0.499872) (layer F.Cu) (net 4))
 (segment (start 182.88 110.49) (end 176.322563 103.932563) (width 0.499872) (layer F.Cu) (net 4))
 (segment (start 182.88 124.46) (end 177.8 129.54) (width 0.499872) (layer F.Cu) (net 6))
 (segment (start 185.42 124.46) (end 182.88 124.46) (width 0.499872) (layer F.Cu) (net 6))
 (segment (start 177.8 130.81) (end 177.8 129.54) (width 0.499872) (layer F.Cu) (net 6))
 (segment (start 184.430051 124.46) (end 185.42 124.46) (width 0.499872) (layer F.Cu) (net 6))
 (segment (start 175.622681 115.65263) (end 184.430051 124.46) (width 0.499872) (layer F.Cu) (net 6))
 (segment (start 170.150063 93.759555) (end 175.622681 99.232173) (width 0.499872) (layer F.Cu) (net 6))
 (segment (start 170.150063 83.849937) (end 170.150063 93.759555) (width 0.499872) (layer F.Cu) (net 6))
 (segment (start 175.622681 99.232173) (end 175.622681 115.65263) (width 0.499872) (layer F.Cu) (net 6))
 (segment (start 171.45 82.55) (end 170.150063 83.849937) (width 0.499872) (layer F.Cu) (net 6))
 (segment (start 199.39 96.52) (end 199.39 121.92) (width 0.499872) (layer F.Cu) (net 12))
 (segment (start 192.970001 73.590001) (end 191.77 72.39) (width 0.3) (layer F.Cu) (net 12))
 (segment (start 192.970001 75.506001) (end 192.970001 73.590001) (width 0.3) (layer F.Cu) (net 12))
 (segment (start 192.346001 76.130001) (end 192.970001 75.506001) (width 0.3) (layer F.Cu) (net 12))
 (segment (start 191.333997 76.130001) (end 192.346001 76.130001) (width 0.3) (layer F.Cu) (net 12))
 (segment (start 190.569999 76.893999) (end 191.333997 76.130001) (width 0.3) (layer F.Cu) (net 12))
 (segment (start 190.569999 78.046001) (end 190.569999 76.893999) (width 0.3) (layer F.Cu) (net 12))
 (segment (start 192.346001 78.670001) (end 191.193999 78.670001) (width 0.3) (layer F.Cu) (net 12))
 (segment (start 199.39 85.714) (end 192.346001 78.670001) (width 0.3) (layer F.Cu) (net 12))
 (segment (start 191.193999 78.670001) (end 190.569999 78.046001) (width 0.3) (layer F.Cu) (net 12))
 (segment (start 199.39 96.52) (end 199.39 85.714) (width 0.3) (layer F.Cu) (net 12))
 (segment (start 185.42 88.9) (end 185.42 96.52) (width 0.499872) (layer F.Cu) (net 2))
 (segment (start 189.23 85.09) (end 185.42 88.9) (width 0.499872) (layer F.Cu) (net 2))
 (segment (start 191.77 85.09) (end 189.23 85.09) (width 0.499872) (layer F.Cu) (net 2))
 (segment (start 181.61 96.52) (end 177.8 100.33) (width 0.499872) (layer F.Cu) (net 2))
 (segment (start 185.42 96.52) (end 181.61 96.52) (width 0.499872) (layer F.Cu) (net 2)))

